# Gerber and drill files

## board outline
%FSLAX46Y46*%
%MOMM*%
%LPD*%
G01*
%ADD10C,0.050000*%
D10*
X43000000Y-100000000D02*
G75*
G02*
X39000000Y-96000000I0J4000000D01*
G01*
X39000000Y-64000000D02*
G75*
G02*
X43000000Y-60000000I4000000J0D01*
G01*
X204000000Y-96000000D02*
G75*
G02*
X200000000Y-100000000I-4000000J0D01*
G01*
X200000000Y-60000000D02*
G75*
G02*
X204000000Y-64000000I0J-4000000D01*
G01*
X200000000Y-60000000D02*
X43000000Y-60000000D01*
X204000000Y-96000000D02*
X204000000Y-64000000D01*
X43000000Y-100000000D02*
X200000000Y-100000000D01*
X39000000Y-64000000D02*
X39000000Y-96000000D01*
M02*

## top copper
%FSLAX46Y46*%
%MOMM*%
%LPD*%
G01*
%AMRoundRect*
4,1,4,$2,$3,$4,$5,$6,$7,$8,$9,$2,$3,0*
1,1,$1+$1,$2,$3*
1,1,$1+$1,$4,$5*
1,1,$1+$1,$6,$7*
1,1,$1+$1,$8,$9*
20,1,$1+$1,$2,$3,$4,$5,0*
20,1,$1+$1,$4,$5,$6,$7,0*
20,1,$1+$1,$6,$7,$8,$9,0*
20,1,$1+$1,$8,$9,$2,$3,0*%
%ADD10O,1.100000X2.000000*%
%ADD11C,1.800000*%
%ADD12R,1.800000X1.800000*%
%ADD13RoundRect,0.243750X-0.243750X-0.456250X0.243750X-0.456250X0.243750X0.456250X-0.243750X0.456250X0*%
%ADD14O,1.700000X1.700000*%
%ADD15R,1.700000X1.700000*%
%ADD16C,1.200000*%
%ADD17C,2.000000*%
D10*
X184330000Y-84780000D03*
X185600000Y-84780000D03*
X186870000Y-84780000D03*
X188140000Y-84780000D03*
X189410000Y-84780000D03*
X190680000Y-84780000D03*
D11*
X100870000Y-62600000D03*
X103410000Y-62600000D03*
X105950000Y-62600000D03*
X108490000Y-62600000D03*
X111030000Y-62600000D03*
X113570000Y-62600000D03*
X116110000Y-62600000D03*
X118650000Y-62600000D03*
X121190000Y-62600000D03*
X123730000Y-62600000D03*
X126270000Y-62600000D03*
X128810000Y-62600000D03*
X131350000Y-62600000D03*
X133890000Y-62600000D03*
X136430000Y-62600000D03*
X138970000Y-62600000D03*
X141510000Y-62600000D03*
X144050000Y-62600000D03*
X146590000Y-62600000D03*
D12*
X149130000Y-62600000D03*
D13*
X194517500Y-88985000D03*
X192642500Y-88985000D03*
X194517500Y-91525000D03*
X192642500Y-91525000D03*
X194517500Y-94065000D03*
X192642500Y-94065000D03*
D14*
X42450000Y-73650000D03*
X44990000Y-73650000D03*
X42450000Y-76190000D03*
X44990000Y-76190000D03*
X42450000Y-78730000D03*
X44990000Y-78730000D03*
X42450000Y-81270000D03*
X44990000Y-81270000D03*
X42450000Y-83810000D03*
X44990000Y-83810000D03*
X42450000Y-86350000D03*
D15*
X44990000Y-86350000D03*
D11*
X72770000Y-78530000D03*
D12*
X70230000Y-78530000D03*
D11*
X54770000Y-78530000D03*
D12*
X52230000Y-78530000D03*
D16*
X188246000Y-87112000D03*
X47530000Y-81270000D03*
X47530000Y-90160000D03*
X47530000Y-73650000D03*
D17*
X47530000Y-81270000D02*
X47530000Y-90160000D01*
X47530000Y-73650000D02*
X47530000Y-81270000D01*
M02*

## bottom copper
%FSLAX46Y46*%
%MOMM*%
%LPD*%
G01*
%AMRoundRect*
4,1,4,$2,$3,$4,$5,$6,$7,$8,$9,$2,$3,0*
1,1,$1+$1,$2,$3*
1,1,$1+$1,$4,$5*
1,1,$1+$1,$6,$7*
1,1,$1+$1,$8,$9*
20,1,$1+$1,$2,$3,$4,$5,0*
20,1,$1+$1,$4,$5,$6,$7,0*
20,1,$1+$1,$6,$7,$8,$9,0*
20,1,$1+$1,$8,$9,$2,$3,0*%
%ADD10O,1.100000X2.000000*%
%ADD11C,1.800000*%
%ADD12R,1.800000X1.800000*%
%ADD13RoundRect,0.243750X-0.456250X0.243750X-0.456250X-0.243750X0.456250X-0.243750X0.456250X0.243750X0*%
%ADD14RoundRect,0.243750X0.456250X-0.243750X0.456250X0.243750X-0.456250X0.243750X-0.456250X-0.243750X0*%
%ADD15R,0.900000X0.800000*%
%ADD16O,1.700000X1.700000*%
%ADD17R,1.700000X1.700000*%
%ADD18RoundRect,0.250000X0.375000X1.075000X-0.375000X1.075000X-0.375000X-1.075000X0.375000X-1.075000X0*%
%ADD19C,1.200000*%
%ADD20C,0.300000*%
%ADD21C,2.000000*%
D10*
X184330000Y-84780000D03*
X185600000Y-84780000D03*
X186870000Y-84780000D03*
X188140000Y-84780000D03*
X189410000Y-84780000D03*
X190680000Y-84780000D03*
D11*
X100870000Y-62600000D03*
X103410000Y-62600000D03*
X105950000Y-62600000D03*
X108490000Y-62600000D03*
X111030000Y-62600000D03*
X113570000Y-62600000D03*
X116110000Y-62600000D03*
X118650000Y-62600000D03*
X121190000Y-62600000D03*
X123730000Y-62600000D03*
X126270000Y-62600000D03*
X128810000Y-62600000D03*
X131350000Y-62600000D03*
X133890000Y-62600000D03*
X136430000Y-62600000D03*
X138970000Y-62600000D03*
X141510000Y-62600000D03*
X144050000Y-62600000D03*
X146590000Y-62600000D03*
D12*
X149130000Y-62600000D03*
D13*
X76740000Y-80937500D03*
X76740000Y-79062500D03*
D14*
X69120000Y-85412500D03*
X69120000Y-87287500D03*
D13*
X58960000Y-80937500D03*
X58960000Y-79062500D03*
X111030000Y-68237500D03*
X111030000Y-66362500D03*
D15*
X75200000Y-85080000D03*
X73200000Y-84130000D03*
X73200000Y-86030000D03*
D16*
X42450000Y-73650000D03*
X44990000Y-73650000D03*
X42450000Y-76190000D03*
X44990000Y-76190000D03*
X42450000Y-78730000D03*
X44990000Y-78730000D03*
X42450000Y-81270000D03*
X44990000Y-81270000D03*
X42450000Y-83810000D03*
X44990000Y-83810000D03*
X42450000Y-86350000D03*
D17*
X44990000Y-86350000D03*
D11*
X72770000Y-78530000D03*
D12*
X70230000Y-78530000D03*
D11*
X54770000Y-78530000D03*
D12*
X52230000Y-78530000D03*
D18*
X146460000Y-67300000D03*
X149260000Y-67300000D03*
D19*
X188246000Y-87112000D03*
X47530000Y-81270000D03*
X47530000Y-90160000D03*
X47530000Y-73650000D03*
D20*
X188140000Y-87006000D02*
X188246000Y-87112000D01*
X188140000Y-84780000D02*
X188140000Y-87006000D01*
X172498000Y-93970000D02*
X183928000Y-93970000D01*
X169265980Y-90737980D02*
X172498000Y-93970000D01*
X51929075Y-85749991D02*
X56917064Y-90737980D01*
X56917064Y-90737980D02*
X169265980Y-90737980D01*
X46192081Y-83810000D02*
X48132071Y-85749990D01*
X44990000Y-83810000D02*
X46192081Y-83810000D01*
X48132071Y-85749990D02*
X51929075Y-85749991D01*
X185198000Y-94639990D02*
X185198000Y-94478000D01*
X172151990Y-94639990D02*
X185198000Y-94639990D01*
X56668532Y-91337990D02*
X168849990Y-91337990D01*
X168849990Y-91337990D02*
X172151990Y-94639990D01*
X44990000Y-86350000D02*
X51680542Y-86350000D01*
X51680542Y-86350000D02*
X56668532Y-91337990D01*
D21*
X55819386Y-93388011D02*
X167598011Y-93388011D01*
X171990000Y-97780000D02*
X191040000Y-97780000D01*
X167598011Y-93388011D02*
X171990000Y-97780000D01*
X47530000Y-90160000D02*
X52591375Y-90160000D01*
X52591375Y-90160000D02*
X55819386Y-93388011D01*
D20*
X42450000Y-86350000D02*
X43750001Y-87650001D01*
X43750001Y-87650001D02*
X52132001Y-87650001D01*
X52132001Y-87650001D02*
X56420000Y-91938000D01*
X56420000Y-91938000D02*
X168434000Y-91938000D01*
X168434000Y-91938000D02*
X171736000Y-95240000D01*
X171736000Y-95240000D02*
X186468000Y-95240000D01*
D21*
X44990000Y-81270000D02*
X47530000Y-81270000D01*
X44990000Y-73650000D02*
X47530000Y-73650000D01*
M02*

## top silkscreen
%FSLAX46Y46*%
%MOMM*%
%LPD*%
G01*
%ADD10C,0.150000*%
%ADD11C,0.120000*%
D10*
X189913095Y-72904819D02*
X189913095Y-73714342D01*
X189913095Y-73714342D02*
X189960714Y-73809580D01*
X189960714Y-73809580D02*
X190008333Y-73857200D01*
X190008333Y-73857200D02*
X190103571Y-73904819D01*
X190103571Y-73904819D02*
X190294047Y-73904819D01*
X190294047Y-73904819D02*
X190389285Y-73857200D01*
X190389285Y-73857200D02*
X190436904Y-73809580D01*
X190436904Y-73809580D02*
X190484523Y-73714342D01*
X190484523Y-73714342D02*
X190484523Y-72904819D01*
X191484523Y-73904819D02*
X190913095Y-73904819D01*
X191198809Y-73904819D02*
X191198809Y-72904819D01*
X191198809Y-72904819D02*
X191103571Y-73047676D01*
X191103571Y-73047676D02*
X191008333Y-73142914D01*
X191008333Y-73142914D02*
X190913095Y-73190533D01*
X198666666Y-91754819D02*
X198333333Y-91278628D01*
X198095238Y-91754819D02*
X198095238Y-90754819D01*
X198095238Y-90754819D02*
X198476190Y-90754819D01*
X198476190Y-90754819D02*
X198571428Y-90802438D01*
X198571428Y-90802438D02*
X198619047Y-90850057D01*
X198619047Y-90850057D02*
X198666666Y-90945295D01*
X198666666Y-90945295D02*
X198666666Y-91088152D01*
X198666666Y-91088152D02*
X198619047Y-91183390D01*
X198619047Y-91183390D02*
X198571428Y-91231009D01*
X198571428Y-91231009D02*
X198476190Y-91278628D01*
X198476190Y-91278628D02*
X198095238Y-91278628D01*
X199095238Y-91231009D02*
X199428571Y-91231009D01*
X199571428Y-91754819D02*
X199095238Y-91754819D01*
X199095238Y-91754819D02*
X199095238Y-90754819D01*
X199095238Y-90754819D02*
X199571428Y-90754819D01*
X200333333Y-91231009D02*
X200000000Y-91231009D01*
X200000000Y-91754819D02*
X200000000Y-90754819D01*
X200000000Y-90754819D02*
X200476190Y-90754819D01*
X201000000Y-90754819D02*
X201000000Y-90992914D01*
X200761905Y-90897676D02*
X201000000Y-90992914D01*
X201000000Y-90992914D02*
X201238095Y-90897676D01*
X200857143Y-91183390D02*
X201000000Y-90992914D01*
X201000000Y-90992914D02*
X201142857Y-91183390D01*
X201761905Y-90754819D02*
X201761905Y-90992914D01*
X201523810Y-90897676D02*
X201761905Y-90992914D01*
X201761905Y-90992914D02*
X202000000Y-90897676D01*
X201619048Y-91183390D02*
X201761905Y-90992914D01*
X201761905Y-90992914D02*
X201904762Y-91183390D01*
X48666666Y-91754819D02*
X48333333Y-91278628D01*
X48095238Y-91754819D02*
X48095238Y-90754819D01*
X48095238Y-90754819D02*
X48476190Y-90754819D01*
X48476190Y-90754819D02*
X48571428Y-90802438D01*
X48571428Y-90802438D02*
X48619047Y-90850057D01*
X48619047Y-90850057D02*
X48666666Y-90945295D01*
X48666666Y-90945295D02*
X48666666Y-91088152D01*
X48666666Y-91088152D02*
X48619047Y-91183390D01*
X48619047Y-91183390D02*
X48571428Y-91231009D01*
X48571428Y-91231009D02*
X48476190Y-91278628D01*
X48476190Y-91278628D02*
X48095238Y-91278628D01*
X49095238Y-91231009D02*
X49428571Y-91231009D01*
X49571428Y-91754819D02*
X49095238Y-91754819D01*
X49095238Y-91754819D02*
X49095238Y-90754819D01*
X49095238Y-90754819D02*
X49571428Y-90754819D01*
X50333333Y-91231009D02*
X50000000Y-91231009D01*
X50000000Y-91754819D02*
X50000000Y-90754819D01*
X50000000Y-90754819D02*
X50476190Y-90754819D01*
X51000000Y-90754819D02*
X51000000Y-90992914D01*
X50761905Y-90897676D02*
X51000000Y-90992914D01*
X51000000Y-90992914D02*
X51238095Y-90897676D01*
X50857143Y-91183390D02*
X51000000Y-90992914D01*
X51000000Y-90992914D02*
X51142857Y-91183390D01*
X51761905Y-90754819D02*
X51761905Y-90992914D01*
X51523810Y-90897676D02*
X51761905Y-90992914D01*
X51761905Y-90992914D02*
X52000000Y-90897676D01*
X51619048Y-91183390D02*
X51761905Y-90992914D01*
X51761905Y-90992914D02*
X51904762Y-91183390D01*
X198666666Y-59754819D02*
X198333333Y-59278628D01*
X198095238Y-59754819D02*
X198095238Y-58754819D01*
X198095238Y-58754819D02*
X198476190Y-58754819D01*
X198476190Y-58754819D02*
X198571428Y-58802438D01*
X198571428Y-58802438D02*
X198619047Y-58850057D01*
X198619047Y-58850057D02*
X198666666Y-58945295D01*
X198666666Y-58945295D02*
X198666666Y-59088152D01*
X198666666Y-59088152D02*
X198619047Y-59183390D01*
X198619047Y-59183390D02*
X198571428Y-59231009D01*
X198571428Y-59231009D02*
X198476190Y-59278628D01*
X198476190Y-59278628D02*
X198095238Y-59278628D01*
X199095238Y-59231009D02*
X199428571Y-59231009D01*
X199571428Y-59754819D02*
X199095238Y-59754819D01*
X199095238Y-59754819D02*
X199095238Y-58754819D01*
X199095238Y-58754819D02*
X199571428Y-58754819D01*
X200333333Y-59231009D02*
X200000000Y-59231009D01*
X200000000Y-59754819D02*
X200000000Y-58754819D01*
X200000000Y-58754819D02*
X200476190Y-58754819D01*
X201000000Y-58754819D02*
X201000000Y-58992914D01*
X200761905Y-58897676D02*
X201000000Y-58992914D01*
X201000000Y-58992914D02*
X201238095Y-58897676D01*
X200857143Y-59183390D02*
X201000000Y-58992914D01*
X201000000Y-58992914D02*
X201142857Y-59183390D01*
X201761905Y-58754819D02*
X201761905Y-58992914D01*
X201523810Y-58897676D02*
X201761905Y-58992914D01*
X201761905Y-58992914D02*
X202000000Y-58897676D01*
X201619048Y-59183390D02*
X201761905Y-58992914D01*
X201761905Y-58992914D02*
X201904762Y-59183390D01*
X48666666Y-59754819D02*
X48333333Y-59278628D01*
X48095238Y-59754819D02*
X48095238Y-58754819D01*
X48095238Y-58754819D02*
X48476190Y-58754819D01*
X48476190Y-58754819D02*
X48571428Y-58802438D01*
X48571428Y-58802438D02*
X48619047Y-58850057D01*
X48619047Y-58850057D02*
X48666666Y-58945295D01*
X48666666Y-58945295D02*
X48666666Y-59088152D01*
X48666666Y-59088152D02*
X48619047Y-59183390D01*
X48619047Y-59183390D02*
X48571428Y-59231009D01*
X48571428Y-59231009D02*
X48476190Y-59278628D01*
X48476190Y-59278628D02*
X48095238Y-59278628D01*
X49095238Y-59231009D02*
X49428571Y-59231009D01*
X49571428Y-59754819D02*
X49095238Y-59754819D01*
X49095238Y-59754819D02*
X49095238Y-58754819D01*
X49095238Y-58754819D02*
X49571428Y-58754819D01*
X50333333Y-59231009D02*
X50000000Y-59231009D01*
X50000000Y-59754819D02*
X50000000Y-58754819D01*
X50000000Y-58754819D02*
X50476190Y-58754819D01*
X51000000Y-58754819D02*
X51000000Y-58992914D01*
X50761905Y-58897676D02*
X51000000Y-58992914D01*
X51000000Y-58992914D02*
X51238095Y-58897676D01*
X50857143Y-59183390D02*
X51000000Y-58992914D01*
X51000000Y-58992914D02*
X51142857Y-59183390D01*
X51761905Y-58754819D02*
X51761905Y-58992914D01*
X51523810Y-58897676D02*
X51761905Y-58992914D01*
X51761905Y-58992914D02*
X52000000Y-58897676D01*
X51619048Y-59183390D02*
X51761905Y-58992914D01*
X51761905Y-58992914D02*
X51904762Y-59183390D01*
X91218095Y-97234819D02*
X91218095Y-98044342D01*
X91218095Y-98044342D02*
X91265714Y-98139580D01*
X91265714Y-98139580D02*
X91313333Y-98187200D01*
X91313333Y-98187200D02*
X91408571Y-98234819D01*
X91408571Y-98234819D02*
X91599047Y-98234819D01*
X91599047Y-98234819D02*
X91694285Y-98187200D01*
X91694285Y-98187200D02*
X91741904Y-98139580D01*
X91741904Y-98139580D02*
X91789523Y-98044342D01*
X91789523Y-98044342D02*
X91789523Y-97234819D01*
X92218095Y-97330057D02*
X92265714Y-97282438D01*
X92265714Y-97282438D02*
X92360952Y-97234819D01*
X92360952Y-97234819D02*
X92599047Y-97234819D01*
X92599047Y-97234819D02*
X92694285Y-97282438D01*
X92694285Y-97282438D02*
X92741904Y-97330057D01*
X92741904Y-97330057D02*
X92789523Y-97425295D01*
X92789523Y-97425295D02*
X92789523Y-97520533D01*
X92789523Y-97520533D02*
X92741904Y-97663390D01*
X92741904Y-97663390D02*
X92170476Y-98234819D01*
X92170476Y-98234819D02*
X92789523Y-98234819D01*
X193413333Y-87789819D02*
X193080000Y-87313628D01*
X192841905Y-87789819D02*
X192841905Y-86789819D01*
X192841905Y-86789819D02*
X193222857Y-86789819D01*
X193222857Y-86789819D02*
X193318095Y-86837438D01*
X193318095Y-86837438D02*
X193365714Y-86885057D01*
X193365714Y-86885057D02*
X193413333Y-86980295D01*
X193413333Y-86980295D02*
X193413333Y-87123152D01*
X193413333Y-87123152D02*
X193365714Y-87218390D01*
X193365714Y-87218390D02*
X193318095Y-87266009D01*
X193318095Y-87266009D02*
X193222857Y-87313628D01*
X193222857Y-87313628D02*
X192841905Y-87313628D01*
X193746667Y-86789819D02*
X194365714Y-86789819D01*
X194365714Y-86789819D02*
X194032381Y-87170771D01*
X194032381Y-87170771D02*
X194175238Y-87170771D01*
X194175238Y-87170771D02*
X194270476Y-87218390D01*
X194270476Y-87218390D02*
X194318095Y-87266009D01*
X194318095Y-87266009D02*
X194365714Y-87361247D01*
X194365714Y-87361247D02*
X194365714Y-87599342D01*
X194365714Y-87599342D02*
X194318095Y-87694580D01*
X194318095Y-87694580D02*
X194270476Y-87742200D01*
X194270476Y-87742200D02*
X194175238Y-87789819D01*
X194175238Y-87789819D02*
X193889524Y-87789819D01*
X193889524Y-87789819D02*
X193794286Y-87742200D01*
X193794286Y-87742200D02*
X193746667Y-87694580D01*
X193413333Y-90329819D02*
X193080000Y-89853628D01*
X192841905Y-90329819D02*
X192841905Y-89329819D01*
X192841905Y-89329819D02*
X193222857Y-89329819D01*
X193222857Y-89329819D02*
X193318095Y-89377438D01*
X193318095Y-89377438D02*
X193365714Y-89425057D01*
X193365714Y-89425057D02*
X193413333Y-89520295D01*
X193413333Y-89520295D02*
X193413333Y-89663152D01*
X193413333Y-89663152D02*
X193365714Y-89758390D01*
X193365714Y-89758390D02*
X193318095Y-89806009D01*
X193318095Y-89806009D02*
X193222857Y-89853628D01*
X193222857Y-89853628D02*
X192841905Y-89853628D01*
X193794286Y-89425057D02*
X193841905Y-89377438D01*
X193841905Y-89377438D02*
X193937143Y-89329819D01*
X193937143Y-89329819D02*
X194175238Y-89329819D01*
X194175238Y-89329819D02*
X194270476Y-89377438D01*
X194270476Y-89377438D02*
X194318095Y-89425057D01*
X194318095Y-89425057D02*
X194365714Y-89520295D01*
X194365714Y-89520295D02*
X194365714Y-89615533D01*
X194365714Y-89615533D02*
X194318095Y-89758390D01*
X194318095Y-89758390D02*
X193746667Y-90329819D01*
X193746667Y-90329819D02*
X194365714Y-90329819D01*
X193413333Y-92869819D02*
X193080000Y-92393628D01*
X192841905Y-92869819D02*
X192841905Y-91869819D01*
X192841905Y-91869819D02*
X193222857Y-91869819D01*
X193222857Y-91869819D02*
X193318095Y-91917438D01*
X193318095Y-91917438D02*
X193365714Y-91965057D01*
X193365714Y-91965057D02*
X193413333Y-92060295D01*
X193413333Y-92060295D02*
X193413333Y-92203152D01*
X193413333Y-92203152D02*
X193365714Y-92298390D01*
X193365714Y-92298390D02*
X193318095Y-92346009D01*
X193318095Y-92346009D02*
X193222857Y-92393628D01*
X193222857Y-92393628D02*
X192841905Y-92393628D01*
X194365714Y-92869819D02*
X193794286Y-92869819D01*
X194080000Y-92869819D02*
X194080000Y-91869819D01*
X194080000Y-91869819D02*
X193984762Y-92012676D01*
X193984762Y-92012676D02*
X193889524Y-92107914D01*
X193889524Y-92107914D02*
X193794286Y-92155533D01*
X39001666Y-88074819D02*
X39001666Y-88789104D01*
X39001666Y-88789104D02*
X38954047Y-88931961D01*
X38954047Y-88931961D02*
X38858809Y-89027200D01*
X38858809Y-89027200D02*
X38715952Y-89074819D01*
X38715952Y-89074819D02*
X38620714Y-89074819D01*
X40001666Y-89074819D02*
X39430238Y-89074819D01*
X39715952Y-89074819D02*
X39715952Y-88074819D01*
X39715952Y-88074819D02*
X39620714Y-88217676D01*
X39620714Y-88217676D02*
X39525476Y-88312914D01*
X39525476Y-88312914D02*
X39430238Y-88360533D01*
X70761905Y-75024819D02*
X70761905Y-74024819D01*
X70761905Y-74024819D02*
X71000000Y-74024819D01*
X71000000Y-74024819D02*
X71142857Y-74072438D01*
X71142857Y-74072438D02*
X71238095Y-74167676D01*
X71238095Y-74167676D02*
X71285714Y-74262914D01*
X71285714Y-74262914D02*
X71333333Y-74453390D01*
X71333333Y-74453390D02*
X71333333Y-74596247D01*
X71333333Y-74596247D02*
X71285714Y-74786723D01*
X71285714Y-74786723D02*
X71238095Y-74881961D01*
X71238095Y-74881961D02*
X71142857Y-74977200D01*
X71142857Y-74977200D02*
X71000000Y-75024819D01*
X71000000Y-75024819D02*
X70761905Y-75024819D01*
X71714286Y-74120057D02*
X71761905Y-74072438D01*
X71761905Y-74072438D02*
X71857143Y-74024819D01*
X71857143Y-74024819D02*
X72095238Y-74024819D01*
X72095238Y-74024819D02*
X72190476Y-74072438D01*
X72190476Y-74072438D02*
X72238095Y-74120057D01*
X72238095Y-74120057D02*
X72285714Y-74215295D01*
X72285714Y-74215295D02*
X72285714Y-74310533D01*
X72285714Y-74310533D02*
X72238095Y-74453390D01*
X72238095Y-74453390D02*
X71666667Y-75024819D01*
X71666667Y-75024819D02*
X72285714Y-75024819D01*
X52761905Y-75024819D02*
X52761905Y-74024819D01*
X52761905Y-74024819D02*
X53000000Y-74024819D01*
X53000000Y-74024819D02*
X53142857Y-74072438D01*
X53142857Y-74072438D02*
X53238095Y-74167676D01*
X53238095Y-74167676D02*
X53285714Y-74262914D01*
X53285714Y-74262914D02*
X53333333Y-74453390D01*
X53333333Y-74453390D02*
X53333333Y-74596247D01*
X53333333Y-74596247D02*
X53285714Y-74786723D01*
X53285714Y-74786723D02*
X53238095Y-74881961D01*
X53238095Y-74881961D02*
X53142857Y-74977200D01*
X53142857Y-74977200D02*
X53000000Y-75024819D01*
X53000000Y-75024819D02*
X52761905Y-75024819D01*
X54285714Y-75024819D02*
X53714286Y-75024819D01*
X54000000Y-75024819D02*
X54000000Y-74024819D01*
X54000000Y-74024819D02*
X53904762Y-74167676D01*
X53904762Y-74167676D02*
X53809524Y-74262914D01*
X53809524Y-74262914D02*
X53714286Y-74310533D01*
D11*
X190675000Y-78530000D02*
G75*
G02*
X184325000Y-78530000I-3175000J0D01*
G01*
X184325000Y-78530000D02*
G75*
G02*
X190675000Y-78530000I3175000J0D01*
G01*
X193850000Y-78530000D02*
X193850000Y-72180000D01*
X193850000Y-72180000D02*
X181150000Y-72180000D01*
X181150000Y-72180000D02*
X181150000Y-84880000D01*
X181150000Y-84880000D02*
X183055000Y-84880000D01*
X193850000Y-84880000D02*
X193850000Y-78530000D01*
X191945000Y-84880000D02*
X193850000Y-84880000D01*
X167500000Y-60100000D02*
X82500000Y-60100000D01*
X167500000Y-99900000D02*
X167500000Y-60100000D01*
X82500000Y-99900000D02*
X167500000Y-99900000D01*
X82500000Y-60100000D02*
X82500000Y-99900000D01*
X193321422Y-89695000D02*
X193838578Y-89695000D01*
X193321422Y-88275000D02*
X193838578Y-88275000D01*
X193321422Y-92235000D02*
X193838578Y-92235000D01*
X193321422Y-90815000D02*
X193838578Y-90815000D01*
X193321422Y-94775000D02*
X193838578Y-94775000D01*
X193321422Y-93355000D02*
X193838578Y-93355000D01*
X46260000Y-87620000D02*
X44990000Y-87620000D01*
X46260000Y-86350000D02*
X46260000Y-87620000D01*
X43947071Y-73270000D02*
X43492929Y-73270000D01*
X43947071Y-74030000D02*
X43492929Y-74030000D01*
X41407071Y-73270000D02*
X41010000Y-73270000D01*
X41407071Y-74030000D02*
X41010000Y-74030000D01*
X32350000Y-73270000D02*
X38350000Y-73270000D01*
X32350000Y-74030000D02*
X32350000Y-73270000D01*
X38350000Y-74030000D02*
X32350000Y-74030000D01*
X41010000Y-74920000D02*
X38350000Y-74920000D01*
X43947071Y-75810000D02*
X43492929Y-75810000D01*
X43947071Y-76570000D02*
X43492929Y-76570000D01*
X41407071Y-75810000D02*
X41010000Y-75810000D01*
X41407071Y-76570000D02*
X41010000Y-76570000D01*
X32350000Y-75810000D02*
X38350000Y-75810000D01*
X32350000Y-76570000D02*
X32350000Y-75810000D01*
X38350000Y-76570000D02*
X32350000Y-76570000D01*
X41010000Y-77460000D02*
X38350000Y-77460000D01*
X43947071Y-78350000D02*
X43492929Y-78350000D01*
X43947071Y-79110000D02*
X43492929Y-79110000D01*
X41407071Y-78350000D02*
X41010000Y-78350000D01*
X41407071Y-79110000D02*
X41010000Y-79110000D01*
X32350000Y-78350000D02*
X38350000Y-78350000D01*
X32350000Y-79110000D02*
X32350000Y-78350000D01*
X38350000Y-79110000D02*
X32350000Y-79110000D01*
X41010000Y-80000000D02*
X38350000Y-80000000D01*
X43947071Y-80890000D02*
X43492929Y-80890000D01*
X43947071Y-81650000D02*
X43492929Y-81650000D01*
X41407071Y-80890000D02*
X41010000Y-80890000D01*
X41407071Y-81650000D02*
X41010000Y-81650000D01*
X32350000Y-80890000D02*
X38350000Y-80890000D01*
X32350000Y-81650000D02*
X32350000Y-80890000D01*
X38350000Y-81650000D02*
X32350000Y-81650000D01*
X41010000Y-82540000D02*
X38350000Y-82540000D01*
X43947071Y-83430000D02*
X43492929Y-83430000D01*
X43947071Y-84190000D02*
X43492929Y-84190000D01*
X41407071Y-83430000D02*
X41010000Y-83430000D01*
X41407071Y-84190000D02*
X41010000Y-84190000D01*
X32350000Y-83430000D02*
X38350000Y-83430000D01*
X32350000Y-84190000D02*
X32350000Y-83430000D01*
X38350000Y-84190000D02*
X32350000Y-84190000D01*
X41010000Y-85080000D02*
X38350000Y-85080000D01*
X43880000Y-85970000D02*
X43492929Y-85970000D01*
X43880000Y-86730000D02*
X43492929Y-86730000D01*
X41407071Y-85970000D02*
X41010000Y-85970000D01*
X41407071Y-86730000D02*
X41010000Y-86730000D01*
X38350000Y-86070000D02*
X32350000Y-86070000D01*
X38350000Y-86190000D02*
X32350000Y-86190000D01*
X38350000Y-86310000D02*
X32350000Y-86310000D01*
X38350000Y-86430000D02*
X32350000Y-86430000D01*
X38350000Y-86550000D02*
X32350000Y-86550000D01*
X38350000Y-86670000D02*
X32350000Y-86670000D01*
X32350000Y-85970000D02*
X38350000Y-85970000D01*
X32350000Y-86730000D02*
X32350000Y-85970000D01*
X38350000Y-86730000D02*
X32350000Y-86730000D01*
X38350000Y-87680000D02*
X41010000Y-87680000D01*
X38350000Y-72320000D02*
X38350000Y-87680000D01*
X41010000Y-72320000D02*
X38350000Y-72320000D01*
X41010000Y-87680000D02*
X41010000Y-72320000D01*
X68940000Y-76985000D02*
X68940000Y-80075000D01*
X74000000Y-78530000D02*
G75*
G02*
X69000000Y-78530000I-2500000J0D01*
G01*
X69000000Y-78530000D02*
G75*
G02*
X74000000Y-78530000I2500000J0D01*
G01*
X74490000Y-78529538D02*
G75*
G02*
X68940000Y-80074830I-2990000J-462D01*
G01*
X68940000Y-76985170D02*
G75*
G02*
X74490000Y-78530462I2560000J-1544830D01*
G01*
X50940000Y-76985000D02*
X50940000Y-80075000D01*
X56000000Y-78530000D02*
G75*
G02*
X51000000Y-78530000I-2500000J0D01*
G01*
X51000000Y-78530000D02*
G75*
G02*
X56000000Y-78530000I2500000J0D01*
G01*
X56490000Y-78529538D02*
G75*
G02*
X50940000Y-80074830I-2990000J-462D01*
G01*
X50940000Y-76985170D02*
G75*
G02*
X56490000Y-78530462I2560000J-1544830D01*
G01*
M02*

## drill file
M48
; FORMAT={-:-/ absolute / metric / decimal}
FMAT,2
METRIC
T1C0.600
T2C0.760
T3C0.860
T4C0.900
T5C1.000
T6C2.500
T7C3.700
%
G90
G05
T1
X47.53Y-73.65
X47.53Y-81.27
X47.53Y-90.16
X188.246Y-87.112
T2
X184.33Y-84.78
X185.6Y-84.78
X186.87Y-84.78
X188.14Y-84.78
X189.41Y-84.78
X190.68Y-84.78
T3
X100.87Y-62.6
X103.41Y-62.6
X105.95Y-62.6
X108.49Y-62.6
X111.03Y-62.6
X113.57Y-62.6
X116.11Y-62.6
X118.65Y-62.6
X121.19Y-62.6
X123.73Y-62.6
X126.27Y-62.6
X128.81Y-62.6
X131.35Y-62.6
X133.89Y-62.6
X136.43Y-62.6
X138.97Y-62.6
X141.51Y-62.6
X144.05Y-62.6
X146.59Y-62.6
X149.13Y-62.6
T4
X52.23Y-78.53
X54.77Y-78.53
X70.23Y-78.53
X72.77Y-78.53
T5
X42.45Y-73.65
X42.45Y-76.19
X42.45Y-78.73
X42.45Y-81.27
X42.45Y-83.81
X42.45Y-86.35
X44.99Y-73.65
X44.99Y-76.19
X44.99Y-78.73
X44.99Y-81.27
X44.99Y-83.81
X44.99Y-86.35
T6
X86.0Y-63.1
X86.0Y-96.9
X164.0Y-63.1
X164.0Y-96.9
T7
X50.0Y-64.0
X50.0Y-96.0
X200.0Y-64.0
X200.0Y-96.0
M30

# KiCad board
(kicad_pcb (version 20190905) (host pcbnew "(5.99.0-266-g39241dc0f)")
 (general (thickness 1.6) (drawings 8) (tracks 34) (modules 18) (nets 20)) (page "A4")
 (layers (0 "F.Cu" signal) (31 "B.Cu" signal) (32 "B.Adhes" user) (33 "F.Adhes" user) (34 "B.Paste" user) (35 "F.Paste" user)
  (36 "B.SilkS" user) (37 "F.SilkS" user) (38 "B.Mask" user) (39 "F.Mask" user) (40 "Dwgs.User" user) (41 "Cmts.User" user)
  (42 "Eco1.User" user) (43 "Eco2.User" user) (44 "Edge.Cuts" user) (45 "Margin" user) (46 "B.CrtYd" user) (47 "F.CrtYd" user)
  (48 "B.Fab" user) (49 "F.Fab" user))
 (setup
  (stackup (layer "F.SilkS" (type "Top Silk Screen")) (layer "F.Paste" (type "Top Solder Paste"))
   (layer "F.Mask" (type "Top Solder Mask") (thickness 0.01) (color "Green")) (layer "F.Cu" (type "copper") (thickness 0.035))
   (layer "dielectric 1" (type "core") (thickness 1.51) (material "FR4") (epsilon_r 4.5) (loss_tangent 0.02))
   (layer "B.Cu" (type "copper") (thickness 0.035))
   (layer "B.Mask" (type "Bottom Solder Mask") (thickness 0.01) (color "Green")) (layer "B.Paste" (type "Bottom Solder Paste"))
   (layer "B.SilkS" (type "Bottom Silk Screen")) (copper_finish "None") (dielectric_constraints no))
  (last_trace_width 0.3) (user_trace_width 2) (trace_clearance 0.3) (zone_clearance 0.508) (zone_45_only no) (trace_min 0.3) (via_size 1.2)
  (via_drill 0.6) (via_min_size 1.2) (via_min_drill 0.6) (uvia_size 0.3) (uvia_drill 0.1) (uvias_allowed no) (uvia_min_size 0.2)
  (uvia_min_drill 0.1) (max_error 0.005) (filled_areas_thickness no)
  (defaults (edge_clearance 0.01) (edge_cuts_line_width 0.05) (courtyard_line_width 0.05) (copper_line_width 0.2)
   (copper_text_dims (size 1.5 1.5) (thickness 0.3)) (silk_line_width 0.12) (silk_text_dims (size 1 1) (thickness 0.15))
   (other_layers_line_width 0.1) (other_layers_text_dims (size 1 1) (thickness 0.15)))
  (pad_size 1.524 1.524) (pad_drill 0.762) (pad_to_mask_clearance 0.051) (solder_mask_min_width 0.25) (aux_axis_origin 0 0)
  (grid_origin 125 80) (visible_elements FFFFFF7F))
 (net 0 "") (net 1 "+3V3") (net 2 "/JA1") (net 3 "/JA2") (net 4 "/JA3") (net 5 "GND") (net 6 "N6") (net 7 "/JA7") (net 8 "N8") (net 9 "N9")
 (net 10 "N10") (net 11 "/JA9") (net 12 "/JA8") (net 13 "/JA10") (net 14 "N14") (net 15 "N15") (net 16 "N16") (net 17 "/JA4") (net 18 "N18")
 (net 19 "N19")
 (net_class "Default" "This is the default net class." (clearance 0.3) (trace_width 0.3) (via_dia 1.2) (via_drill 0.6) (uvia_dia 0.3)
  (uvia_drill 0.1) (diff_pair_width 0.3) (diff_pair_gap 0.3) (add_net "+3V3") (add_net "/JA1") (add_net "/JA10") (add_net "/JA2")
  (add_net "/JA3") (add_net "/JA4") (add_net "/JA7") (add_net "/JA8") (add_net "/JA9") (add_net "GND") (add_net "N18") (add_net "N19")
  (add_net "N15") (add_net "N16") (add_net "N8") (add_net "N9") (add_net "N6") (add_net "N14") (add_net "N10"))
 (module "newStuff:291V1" (layer "F.Cu") (at 187.5 78.53)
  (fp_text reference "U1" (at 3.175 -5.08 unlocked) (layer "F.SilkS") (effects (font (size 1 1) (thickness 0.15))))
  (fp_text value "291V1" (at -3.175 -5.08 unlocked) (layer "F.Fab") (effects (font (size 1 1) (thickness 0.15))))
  (fp_circle (center 0 0) (end 3.175 0) (layer "F.SilkS") (width 0.12))
  (fp_line (start 6.35 0) (end 6.35 -6.35) (layer "F.SilkS") (width 0.12))
  (fp_line (start 6.35 -6.35) (end -6.35 -6.35) (layer "F.SilkS") (width 0.12))
  (fp_line (start -6.35 -6.35) (end -6.35 6.35) (layer "F.SilkS") (width 0.12))
  (fp_line (start -6.35 6.35) (end -4.445 6.35) (layer "F.SilkS") (width 0.12))
  (fp_line (start 6.35 6.35) (end 6.35 0) (layer "F.SilkS") (width 0.12))
  (fp_line (start 4.445 6.35) (end 6.35 6.35) (layer "F.SilkS") (width 0.12))
  (pad "6" thru_hole oval (at -3.17 6.25) (size 1.1 2) (drill 0.76) (layers *.Cu *.Mask) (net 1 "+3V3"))
  (pad "5" thru_hole oval (at -1.9 6.25) (size 1.1 2) (drill 0.76) (layers *.Cu *.Mask) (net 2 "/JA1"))
  (pad "4" thru_hole oval (at -0.63 6.25) (size 1.1 2) (drill 0.76) (layers *.Cu *.Mask) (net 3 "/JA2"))
  (pad "3" thru_hole oval (at 0.64 6.25) (size 1.1 2) (drill 0.76) (layers *.Cu *.Mask) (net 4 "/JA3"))
  (pad "2" thru_hole oval (at 1.91 6.25) (size 1.1 2) (drill 0.76) (layers *.Cu *.Mask) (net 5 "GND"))
  (pad "1" thru_hole oval (at 3.18 6.25) (size 1.1 2) (drill 0.76) (layers *.Cu *.Mask) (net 5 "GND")))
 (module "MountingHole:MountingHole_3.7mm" (layer "F.Cu") (at 200 96)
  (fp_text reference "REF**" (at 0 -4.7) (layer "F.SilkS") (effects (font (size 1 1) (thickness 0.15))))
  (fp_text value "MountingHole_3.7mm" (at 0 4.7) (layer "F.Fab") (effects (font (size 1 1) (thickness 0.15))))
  (pad "1" np_thru_hole circle (at 0 0) (size 3.7 3.7) (drill 3.7) (layers *.Cu *.Mask)))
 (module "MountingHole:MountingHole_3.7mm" (layer "F.Cu") (at 50 96)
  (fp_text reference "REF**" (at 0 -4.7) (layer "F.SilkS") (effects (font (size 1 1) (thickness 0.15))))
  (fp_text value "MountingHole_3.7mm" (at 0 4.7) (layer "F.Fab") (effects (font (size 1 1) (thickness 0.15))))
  (pad "1" np_thru_hole circle (at 0 0) (size 3.7 3.7) (drill 3.7) (layers *.Cu *.Mask)))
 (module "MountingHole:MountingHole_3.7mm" (layer "F.Cu") (at 200 64)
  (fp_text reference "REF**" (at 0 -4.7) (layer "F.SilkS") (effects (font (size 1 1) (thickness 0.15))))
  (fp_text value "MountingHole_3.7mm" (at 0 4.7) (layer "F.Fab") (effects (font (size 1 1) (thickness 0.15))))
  (pad "1" np_thru_hole circle (at 0 0) (size 3.7 3.7) (drill 3.7) (layers *.Cu *.Mask)))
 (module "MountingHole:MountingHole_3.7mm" (layer "F.Cu") (at 50 64)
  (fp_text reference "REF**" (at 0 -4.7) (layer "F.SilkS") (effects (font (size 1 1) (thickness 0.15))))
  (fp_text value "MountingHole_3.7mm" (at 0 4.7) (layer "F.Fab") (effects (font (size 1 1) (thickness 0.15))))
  (pad "1" np_thru_hole circle (at 0 0) (size 3.7 3.7) (drill 3.7) (layers *.Cu *.Mask)))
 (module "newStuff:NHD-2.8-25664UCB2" (layer "F.Cu") (at 125 80)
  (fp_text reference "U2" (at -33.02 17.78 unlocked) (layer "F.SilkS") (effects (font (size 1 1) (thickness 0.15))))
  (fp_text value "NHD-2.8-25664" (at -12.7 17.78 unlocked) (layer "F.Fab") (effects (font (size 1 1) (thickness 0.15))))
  (fp_line (start 42.5 -19.9) (end -42.5 -19.9) (layer "F.SilkS") (width 0.12))
  (fp_line (start 42.5 19.9) (end 42.5 -19.9) (layer "F.SilkS") (width 0.12))
  (fp_line (start -42.5 19.9) (end 42.5 19.9) (layer "F.SilkS") (width 0.12))
  (fp_line (start -42.5 -19.9) (end -42.5 19.9) (layer "F.SilkS") (width 0.12))
  (pad "20" thru_hole circle (at -24.13 -17.4) (size 1.8 1.8) (drill 0.86) (layers *.Cu *.Mask) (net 5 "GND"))
  (pad "19" thru_hole circle (at -21.59 -17.4) (size 1.8 1.8) (drill 0.86) (layers *.Cu *.Mask) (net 5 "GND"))
  (pad "18" thru_hole circle (at -19.05 -17.4) (size 1.8 1.8) (drill 0.86) (layers *.Cu *.Mask) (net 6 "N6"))
  (pad "17" thru_hole circle (at -16.51 -17.4) (size 1.8 1.8) (drill 0.86) (layers *.Cu *.Mask) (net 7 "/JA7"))
  (pad "16" thru_hole circle (at -13.97 -17.4) (size 1.8 1.8) (drill 0.86) (layers *.Cu *.Mask) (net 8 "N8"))
  (pad "15" thru_hole circle (at -11.43 -17.4) (size 1.8 1.8) (drill 0.86) (layers *.Cu *.Mask) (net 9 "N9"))
  (pad "14" thru_hole circle (at -8.89 -17.4) (size 1.8 1.8) (drill 0.86) (layers *.Cu *.Mask) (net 5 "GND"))
  (pad "13" thru_hole circle (at -6.35 -17.4) (size 1.8 1.8) (drill 0.86) (layers *.Cu *.Mask) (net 5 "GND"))
  (pad "12" thru_hole circle (at -3.81 -17.4) (size 1.8 1.8) (drill 0.86) (layers *.Cu *.Mask) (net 5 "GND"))
  (pad "11" thru_hole circle (at -1.27 -17.4) (size 1.8 1.8) (drill 0.86) (layers *.Cu *.Mask) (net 5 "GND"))
  (pad "10" thru_hole circle (at 1.27 -17.4) (size 1.8 1.8) (drill 0.86) (layers *.Cu *.Mask) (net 5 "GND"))
  (pad "9" thru_hole circle (at 3.81 -17.4) (size 1.8 1.8) (drill 0.86) (layers *.Cu *.Mask) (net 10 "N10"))
  (pad "8" thru_hole circle (at 6.35 -17.4) (size 1.8 1.8) (drill 0.86) (layers *.Cu *.Mask) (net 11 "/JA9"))
  (pad "7" thru_hole circle (at 8.89 -17.4) (size 1.8 1.8) (drill 0.86) (layers *.Cu *.Mask) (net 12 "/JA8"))
  (pad "6" thru_hole circle (at 11.43 -17.4) (size 1.8 1.8) (drill 0.86) (layers *.Cu *.Mask) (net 5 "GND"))
  (pad "5" thru_hole circle (at 13.97 -17.4) (size 1.8 1.8) (drill 0.86) (layers *.Cu *.Mask) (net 5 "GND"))
  (pad "4" thru_hole circle (at 16.51 -17.4) (size 1.8 1.8) (drill 0.86) (layers *.Cu *.Mask) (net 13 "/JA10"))
  (pad "3" thru_hole circle (at 19.05 -17.4) (size 1.8 1.8) (drill 0.86) (layers *.Cu *.Mask) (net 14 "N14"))
  (pad "2" thru_hole circle (at 21.59 -17.4) (size 1.8 1.8) (drill 0.86) (layers *.Cu *.Mask) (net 5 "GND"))
  (pad "1" thru_hole rect (at 24.13 -17.4) (size 1.8 1.8) (drill 0.86) (layers *.Cu *.Mask) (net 1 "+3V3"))
  (pad "" np_thru_hole circle (at -39 -16.9) (size 2.5 2.5) (drill 2.5) (layers *.Cu *.Mask))
  (pad "" np_thru_hole circle (at -39 16.9) (size 2.5 2.5) (drill 2.5) (layers *.Cu *.Mask))
  (pad "" np_thru_hole circle (at 39 -16.9) (size 2.5 2.5) (drill 2.5) (layers *.Cu *.Mask))
  (pad "" np_thru_hole circle (at 39 16.9) (size 2.5 2.5) (drill 2.5) (layers *.Cu *.Mask)))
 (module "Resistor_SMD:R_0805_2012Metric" (layer "B.Cu") (at 76.74 80 -90)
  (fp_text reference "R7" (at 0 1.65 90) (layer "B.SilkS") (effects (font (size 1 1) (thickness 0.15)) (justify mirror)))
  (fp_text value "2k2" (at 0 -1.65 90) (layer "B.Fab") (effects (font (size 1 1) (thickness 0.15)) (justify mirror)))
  (pad "2" smd roundrect (at 0.9375 0 270) (size 0.975 1.4) (layers "B.Cu" "B.Paste" "B.Mask") (roundrect_rratio 0.25) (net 1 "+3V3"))
  (pad "1" smd roundrect (at -0.9375 0 270) (size 0.975 1.4) (layers "B.Cu" "B.Paste" "B.Mask") (roundrect_rratio 0.25) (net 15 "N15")))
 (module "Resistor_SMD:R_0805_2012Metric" (layer "B.Cu") (at 69.12 86.35 90)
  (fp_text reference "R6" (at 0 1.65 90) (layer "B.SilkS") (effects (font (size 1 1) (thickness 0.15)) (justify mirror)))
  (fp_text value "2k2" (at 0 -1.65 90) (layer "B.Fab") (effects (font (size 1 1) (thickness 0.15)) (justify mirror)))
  (pad "2" smd roundrect (at 0.9375 0 90) (size 0.975 1.4) (layers "B.Cu" "B.Paste" "B.Mask") (roundrect_rratio 0.25) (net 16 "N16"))
  (pad "1" smd roundrect (at -0.9375 0 90) (size 0.975 1.4) (layers "B.Cu" "B.Paste" "B.Mask") (roundrect_rratio 0.25) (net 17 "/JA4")))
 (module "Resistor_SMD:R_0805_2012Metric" (layer "B.Cu") (at 58.96 80 -90)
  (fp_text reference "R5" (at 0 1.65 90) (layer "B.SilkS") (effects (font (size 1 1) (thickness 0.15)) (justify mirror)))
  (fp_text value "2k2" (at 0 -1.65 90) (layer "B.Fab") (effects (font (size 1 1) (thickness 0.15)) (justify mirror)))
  (pad "2" smd roundrect (at 0.9375 0 270) (size 0.975 1.4) (layers "B.Cu" "B.Paste" "B.Mask") (roundrect_rratio 0.25) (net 1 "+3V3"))
  (pad "1" smd roundrect (at -0.9375 0 270) (size 0.975 1.4) (layers "B.Cu" "B.Paste" "B.Mask") (roundrect_rratio 0.25) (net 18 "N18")))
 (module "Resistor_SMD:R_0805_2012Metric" (layer "B.Cu") (at 111.03 67.3 -90)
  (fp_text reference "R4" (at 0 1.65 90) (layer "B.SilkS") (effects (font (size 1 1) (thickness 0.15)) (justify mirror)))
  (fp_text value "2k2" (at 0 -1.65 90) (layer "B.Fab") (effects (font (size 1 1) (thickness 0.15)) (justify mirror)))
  (pad "2" smd roundrect (at 0.9375 0 270) (size 0.975 1.4) (layers "B.Cu" "B.Paste" "B.Mask") (roundrect_rratio 0.25) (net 1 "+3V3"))
  (pad "1" smd roundrect (at -0.9375 0 270) (size 0.975 1.4) (layers "B.Cu" "B.Paste" "B.Mask") (roundrect_rratio 0.25) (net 8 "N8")))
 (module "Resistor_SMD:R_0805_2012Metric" (layer "F.Cu") (at 193.58 88.985)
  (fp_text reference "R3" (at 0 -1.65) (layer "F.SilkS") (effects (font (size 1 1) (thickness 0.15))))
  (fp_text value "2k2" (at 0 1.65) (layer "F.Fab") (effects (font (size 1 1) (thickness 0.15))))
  (fp_line (start -0.258578 0.71) (end 0.258578 0.71) (layer "F.SilkS") (width 0.12))
  (fp_line (start -0.258578 -0.71) (end 0.258578 -0.71) (layer "F.SilkS") (width 0.12))
  (pad "2" smd roundrect (at 0.9375 0) (size 0.975 1.4) (layers "F.Cu" "F.Paste" "F.Mask") (roundrect_rratio 0.25) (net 1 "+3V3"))
  (pad "1" smd roundrect (at -0.9375 0) (size 0.975 1.4) (layers "F.Cu" "F.Paste" "F.Mask") (roundrect_rratio 0.25) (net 4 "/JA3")))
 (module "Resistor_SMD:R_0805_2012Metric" (layer "F.Cu") (at 193.58 91.525)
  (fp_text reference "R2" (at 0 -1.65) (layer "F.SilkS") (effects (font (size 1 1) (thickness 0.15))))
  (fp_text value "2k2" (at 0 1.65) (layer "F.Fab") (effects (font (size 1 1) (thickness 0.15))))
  (fp_line (start -0.258578 0.71) (end 0.258578 0.71) (layer "F.SilkS") (width 0.12))
  (fp_line (start -0.258578 -0.71) (end 0.258578 -0.71) (layer "F.SilkS") (width 0.12))
  (pad "2" smd roundrect (at 0.9375 0) (size 0.975 1.4) (layers "F.Cu" "F.Paste" "F.Mask") (roundrect_rratio 0.25) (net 1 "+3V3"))
  (pad "1" smd roundrect (at -0.9375 0) (size 0.975 1.4) (layers "F.Cu" "F.Paste" "F.Mask") (roundrect_rratio 0.25) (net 3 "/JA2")))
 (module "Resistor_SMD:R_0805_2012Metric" (layer "F.Cu") (at 193.58 94.065)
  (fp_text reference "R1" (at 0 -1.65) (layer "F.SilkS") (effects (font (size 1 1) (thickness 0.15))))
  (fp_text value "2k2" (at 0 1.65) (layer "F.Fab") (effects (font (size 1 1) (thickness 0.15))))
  (fp_line (start -0.258578 0.71) (end 0.258578 0.71) (layer "F.SilkS") (width 0.12))
  (fp_line (start -0.258578 -0.71) (end 0.258578 -0.71) (layer "F.SilkS") (width 0.12))
  (pad "2" smd roundrect (at 0.9375 0) (size 0.975 1.4) (layers "F.Cu" "F.Paste" "F.Mask") (roundrect_rratio 0.25) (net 1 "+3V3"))
  (pad "1" smd roundrect (at -0.9375 0) (size 0.975 1.4) (layers "F.Cu" "F.Paste" "F.Mask") (roundrect_rratio 0.25) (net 2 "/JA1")))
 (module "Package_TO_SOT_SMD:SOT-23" (layer "B.Cu") (at 74.2 85.08)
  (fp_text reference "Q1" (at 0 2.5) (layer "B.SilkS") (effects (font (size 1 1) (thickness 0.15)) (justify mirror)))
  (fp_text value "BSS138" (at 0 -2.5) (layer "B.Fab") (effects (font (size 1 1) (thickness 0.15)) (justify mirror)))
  (pad "3" smd rect (at 1 0) (size 0.9 0.8) (layers "B.Cu" "B.Paste" "B.Mask") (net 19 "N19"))
  (pad "2" smd rect (at -1 -0.95) (size 0.9 0.8) (layers "B.Cu" "B.Paste" "B.Mask") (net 5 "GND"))
  (pad "1" smd rect (at -1 0.95) (size 0.9 0.8) (layers "B.Cu" "B.Paste" "B.Mask") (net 16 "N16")))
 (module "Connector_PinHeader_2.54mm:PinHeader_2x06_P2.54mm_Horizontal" (layer "F.Cu") (at 44.99 86.35 180)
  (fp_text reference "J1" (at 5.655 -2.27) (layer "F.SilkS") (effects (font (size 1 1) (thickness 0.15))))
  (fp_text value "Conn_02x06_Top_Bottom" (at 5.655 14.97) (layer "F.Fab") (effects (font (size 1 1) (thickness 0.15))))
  (fp_line (start -1.27 -1.27) (end 0 -1.27) (layer "F.SilkS") (width 0.12))
  (fp_line (start -1.27 0) (end -1.27 -1.27) (layer "F.SilkS") (width 0.12))
  (fp_line (start 1.042929 13.08) (end 1.497071 13.08) (layer "F.SilkS") (width 0.12))
  (fp_line (start 1.042929 12.32) (end 1.497071 12.32) (layer "F.SilkS") (width 0.12))
  (fp_line (start 3.582929 13.08) (end 3.98 13.08) (layer "F.SilkS") (width 0.12))
  (fp_line (start 3.582929 12.32) (end 3.98 12.32) (layer "F.SilkS") (width 0.12))
  (fp_line (start 12.64 13.08) (end 6.64 13.08) (layer "F.SilkS") (width 0.12))
  (fp_line (start 12.64 12.32) (end 12.64 13.08) (layer "F.SilkS") (width 0.12))
  (fp_line (start 6.64 12.32) (end 12.64 12.32) (layer "F.SilkS") (width 0.12))
  (fp_line (start 3.98 11.43) (end 6.64 11.43) (layer "F.SilkS") (width 0.12))
  (fp_line (start 1.042929 10.54) (end 1.497071 10.54) (layer "F.SilkS") (width 0.12))
  (fp_line (start 1.042929 9.78) (end 1.497071 9.78) (layer "F.SilkS") (width 0.12))
  (fp_line (start 3.582929 10.54) (end 3.98 10.54) (layer "F.SilkS") (width 0.12))
  (fp_line (start 3.582929 9.78) (end 3.98 9.78) (layer "F.SilkS") (width 0.12))
  (fp_line (start 12.64 10.54) (end 6.64 10.54) (layer "F.SilkS") (width 0.12))
  (fp_line (start 12.64 9.78) (end 12.64 10.54) (layer "F.SilkS") (width 0.12))
  (fp_line (start 6.64 9.78) (end 12.64 9.78) (layer "F.SilkS") (width 0.12))
  (fp_line (start 3.98 8.89) (end 6.64 8.89) (layer "F.SilkS") (width 0.12))
  (fp_line (start 1.042929 8) (end 1.497071 8) (layer "F.SilkS") (width 0.12))
  (fp_line (start 1.042929 7.24) (end 1.497071 7.24) (layer "F.SilkS") (width 0.12))
  (fp_line (start 3.582929 8) (end 3.98 8) (layer "F.SilkS") (width 0.12))
  (fp_line (start 3.582929 7.24) (end 3.98 7.24) (layer "F.SilkS") (width 0.12))
  (fp_line (start 12.64 8) (end 6.64 8) (layer "F.SilkS") (width 0.12))
  (fp_line (start 12.64 7.24) (end 12.64 8) (layer "F.SilkS") (width 0.12))
  (fp_line (start 6.64 7.24) (end 12.64 7.24) (layer "F.SilkS") (width 0.12))
  (fp_line (start 3.98 6.35) (end 6.64 6.35) (layer "F.SilkS") (width 0.12))
  (fp_line (start 1.042929 5.46) (end 1.497071 5.46) (layer "F.SilkS") (width 0.12))
  (fp_line (start 1.042929 4.7) (end 1.497071 4.7) (layer "F.SilkS") (width 0.12))
  (fp_line (start 3.582929 5.46) (end 3.98 5.46) (layer "F.SilkS") (width 0.12))
  (fp_line (start 3.582929 4.7) (end 3.98 4.7) (layer "F.SilkS") (width 0.12))
  (fp_line (start 12.64 5.46) (end 6.64 5.46) (layer "F.SilkS") (width 0.12))
  (fp_line (start 12.64 4.7) (end 12.64 5.46) (layer "F.SilkS") (width 0.12))
  (fp_line (start 6.64 4.7) (end 12.64 4.7) (layer "F.SilkS") (width 0.12))
  (fp_line (start 3.98 3.81) (end 6.64 3.81) (layer "F.SilkS") (width 0.12))
  (fp_line (start 1.042929 2.92) (end 1.497071 2.92) (layer "F.SilkS") (width 0.12))
  (fp_line (start 1.042929 2.16) (end 1.497071 2.16) (layer "F.SilkS") (width 0.12))
  (fp_line (start 3.582929 2.92) (end 3.98 2.92) (layer "F.SilkS") (width 0.12))
  (fp_line (start 3.582929 2.16) (end 3.98 2.16) (layer "F.SilkS") (width 0.12))
  (fp_line (start 12.64 2.92) (end 6.64 2.92) (layer "F.SilkS") (width 0.12))
  (fp_line (start 12.64 2.16) (end 12.64 2.92) (layer "F.SilkS") (width 0.12))
  (fp_line (start 6.64 2.16) (end 12.64 2.16) (layer "F.SilkS") (width 0.12))
  (fp_line (start 3.98 1.27) (end 6.64 1.27) (layer "F.SilkS") (width 0.12))
  (fp_line (start 1.11 0.38) (end 1.497071 0.38) (layer "F.SilkS") (width 0.12))
  (fp_line (start 1.11 -0.38) (end 1.497071 -0.38) (layer "F.SilkS") (width 0.12))
  (fp_line (start 3.582929 0.38) (end 3.98 0.38) (layer "F.SilkS") (width 0.12))
  (fp_line (start 3.582929 -0.38) (end 3.98 -0.38) (layer "F.SilkS") (width 0.12))
  (fp_line (start 6.64 0.28) (end 12.64 0.28) (layer "F.SilkS") (width 0.12))
  (fp_line (start 6.64 0.16) (end 12.64 0.16) (layer "F.SilkS") (width 0.12))
  (fp_line (start 6.64 0.04) (end 12.64 0.04) (layer "F.SilkS") (width 0.12))
  (fp_line (start 6.64 -0.08) (end 12.64 -0.08) (layer "F.SilkS") (width 0.12))
  (fp_line (start 6.64 -0.2) (end 12.64 -0.2) (layer "F.SilkS") (width 0.12))
  (fp_line (start 6.64 -0.32) (end 12.64 -0.32) (layer "F.SilkS") (width 0.12))
  (fp_line (start 12.64 0.38) (end 6.64 0.38) (layer "F.SilkS") (width 0.12))
  (fp_line (start 12.64 -0.38) (end 12.64 0.38) (layer "F.SilkS") (width 0.12))
  (fp_line (start 6.64 -0.38) (end 12.64 -0.38) (layer "F.SilkS") (width 0.12))
  (fp_line (start 6.64 -1.33) (end 3.98 -1.33) (layer "F.SilkS") (width 0.12))
  (fp_line (start 6.64 14.03) (end 6.64 -1.33) (layer "F.SilkS") (width 0.12))
  (fp_line (start 3.98 14.03) (end 6.64 14.03) (layer "F.SilkS") (width 0.12))
  (fp_line (start 3.98 -1.33) (end 3.98 14.03) (layer "F.SilkS") (width 0.12))
  (pad "12" thru_hole oval (at 2.54 12.7 180) (size 1.7 1.7) (drill 1) (layers *.Cu *.Mask) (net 5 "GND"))
  (pad "11" thru_hole oval (at 0 12.7 180) (size 1.7 1.7) (drill 1) (layers *.Cu *.Mask) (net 1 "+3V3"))
  (pad "10" thru_hole oval (at 2.54 10.16 180) (size 1.7 1.7) (drill 1) (layers *.Cu *.Mask) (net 13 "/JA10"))
  (pad "9" thru_hole oval (at 0 10.16 180) (size 1.7 1.7) (drill 1) (layers *.Cu *.Mask) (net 11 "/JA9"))
  (pad "8" thru_hole oval (at 2.54 7.62 180) (size 1.7 1.7) (drill 1) (layers *.Cu *.Mask) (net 12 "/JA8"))
  (pad "7" thru_hole oval (at 0 7.62 180) (size 1.7 1.7) (drill 1) (layers *.Cu *.Mask) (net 7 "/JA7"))
  (pad "6" thru_hole oval (at 2.54 5.08 180) (size 1.7 1.7) (drill 1) (layers *.Cu *.Mask) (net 5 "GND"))
  (pad "5" thru_hole oval (at 0 5.08 180) (size 1.7 1.7) (drill 1) (layers *.Cu *.Mask) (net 1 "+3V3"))
  (pad "4" thru_hole oval (at 2.54 2.54 180) (size 1.7 1.7) (drill 1) (layers *.Cu *.Mask) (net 17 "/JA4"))
  (pad "3" thru_hole oval (at 0 2.54 180) (size 1.7 1.7) (drill 1) (layers *.Cu *.Mask) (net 4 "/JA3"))
  (pad "2" thru_hole oval (at 2.54 0 180) (size 1.7 1.7) (drill 1) (layers *.Cu *.Mask) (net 3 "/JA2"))
  (pad "1" thru_hole rect (at 0 0 180) (size 1.7 1.7) (drill 1) (layers *.Cu *.Mask) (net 2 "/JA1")))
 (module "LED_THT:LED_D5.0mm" (layer "F.Cu") (at 70.23 78.53)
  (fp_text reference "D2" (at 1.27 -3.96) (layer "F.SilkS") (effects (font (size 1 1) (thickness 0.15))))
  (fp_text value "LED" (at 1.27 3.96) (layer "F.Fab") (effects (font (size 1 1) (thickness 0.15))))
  (fp_line (start -1.29 -1.545) (end -1.29 1.545) (layer "F.SilkS") (width 0.12))
  (fp_circle (center 1.27 0) (end 3.77 0) (layer "F.SilkS") (width 0.12))
  (fp_arc (start 1.27 0) (end -1.29 1.54483) (angle -148.9) (layer "F.SilkS") (width 0.12))
  (fp_arc (start 1.27 0) (end -1.29 -1.54483) (angle 148.9) (layer "F.SilkS") (width 0.12))
  (pad "2" thru_hole circle (at 2.54 0) (size 1.8 1.8) (drill 0.9) (layers *.Cu *.Mask) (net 15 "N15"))
  (pad "1" thru_hole rect (at 0 0) (size 1.8 1.8) (drill 0.9) (layers *.Cu *.Mask) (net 19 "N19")))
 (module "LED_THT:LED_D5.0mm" (layer "F.Cu") (at 52.23 78.53)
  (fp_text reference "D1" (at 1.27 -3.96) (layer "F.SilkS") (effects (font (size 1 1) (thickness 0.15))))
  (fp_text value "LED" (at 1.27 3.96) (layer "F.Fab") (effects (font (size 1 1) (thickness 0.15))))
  (fp_line (start -1.29 -1.545) (end -1.29 1.545) (layer "F.SilkS") (width 0.12))
  (fp_circle (center 1.27 0) (end 3.77 0) (layer "F.SilkS") (width 0.12))
  (fp_arc (start 1.27 0) (end -1.29 1.54483) (angle -148.9) (layer "F.SilkS") (width 0.12))
  (fp_arc (start 1.27 0) (end -1.29 -1.54483) (angle 148.9) (layer "F.SilkS") (width 0.12))
  (pad "2" thru_hole circle (at 2.54 0) (size 1.8 1.8) (drill 0.9) (layers *.Cu *.Mask) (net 18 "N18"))
  (pad "1" thru_hole rect (at 0 0) (size 1.8 1.8) (drill 0.9) (layers *.Cu *.Mask) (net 5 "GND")))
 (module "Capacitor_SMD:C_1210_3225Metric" (layer "B.Cu") (at 147.86 67.3 180)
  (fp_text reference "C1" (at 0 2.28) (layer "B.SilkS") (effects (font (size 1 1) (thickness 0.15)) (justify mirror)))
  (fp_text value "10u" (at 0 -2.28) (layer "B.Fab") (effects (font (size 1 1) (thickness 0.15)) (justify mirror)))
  (pad "2" smd roundrect (at 1.4 0 180) (size 1.25 2.65) (layers "B.Cu" "B.Paste" "B.Mask") (roundrect_rratio 0.2) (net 5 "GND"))
  (pad "1" smd roundrect (at -1.4 0 180) (size 1.25 2.65) (layers "B.Cu" "B.Paste" "B.Mask") (roundrect_rratio 0.2) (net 1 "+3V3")))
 (gr_arc (start 43 96) (end 39 96) (angle -90) (layer "Edge.Cuts") (width 0.05))
 (gr_arc (start 43 64) (end 43 60) (angle -90) (layer "Edge.Cuts") (width 0.05))
 (gr_arc (start 200 96) (end 200 100) (angle -90) (layer "Edge.Cuts") (width 0.05))
 (gr_arc (start 200 64) (end 204 64) (angle -90) (layer "Edge.Cuts") (width 0.05))
 (gr_line (start 200 60) (end 43 60) (layer "Edge.Cuts") (width 0.05))
 (gr_line (start 204 96) (end 204 64) (layer "Edge.Cuts") (width 0.05))
 (gr_line (start 43 100) (end 200 100) (layer "Edge.Cuts") (width 0.05))
 (gr_line (start 39 64) (end 39 96) (layer "Edge.Cuts") (width 0.05))
 (segment (start 188.14 87.006) (end 188.246 87.112) (width 0.3) (layer "B.Cu") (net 4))
 (segment (start 188.14 84.78) (end 188.14 87.006) (width 0.3) (layer "B.Cu") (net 4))
 (via (at 188.246 87.112) (size 1.2) (drill 0.6) (layers "F.Cu" "B.Cu") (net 4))
 (segment (start 172.498 93.97) (end 183.928 93.97) (width 0.3) (layer "B.Cu") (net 4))
 (segment (start 169.26598 90.73798) (end 172.498 93.97) (width 0.3) (layer "B.Cu") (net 4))
 (segment (start 51.929075 85.749991) (end 56.917064 90.73798) (width 0.3) (layer "B.Cu") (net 4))
 (segment (start 56.917064 90.73798) (end 169.26598 90.73798) (width 0.3) (layer "B.Cu") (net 4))
 (segment (start 46.192081 83.81) (end 48.132071 85.74999) (width 0.3) (layer "B.Cu") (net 4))
 (segment (start 44.99 83.81) (end 46.192081 83.81) (width 0.3) (layer "B.Cu") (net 4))
 (segment (start 48.132071 85.74999) (end 51.929075 85.749991) (width 0.3) (layer "B.Cu") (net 4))
 (segment (start 185.198 94.63999) (end 185.198 94.478) (width 0.3) (layer "B.Cu") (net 2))
 (segment (start 172.15199 94.63999) (end 185.198 94.63999) (width 0.3) (layer "B.Cu") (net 2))
 (segment (start 56.668532 91.33799) (end 168.84999 91.33799) (width 0.3) (layer "B.Cu") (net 2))
 (segment (start 168.84999 91.33799) (end 172.15199 94.63999) (width 0.3) (layer "B.Cu") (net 2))
 (segment (start 44.99 86.35) (end 51.680542 86.35) (width 0.3) (layer "B.Cu") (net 2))
 (segment (start 51.680542 86.35) (end 56.668532 91.33799) (width 0.3) (layer "B.Cu") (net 2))
 (segment (start 55.819386 93.388011) (end 167.598011 93.388011) (width 2) (layer "B.Cu") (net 1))
 (segment (start 171.99 97.78) (end 191.04 97.78) (width 2) (layer "B.Cu") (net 1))
 (segment (start 167.598011 93.388011) (end 171.99 97.78) (width 2) (layer "B.Cu") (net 1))
 (segment (start 47.53 90.16) (end 52.591375 90.16) (width 2) (layer "B.Cu") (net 1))
 (segment (start 52.591375 90.16) (end 55.819386 93.388011) (width 2) (layer "B.Cu") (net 1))
 (segment (start 42.45 86.35) (end 43.750001 87.650001) (width 0.3) (layer "B.Cu") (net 3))
 (segment (start 43.750001 87.650001) (end 52.132001 87.650001) (width 0.3) (layer "B.Cu") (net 3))
 (segment (start 52.132001 87.650001) (end 56.42 91.938) (width 0.3) (layer "B.Cu") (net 3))
 (segment (start 56.42 91.938) (end 168.434 91.938) (width 0.3) (layer "B.Cu") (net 3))
 (segment (start 168.434 91.938) (end 171.736 95.24) (width 0.3) (layer "B.Cu") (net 3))
 (segment (start 171.736 95.24) (end 186.468 95.24) (width 0.3) (layer "B.Cu") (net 3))
 (segment (start 47.53 81.27) (end 47.53 90.16) (width 2) (layer "F.Cu") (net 1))
 (segment (start 47.53 73.65) (end 47.53 81.27) (width 2) (layer "F.Cu") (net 1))
 (segment (start 44.99 81.27) (end 47.53 81.27) (width 2) (layer "B.Cu") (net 1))
 (via (at 47.53 81.27) (size 1.2) (drill 0.6) (layers "F.Cu" "B.Cu") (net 1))
 (via (at 47.53 90.16) (size 1.2) (drill 0.6) (layers "F.Cu" "B.Cu") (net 1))
 (segment (start 44.99 73.65) (end 47.53 73.65) (width 2) (layer "B.Cu") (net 1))
 (via (at 47.53 73.65) (size 1.2) (drill 0.6) (layers "F.Cu" "B.Cu") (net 1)))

